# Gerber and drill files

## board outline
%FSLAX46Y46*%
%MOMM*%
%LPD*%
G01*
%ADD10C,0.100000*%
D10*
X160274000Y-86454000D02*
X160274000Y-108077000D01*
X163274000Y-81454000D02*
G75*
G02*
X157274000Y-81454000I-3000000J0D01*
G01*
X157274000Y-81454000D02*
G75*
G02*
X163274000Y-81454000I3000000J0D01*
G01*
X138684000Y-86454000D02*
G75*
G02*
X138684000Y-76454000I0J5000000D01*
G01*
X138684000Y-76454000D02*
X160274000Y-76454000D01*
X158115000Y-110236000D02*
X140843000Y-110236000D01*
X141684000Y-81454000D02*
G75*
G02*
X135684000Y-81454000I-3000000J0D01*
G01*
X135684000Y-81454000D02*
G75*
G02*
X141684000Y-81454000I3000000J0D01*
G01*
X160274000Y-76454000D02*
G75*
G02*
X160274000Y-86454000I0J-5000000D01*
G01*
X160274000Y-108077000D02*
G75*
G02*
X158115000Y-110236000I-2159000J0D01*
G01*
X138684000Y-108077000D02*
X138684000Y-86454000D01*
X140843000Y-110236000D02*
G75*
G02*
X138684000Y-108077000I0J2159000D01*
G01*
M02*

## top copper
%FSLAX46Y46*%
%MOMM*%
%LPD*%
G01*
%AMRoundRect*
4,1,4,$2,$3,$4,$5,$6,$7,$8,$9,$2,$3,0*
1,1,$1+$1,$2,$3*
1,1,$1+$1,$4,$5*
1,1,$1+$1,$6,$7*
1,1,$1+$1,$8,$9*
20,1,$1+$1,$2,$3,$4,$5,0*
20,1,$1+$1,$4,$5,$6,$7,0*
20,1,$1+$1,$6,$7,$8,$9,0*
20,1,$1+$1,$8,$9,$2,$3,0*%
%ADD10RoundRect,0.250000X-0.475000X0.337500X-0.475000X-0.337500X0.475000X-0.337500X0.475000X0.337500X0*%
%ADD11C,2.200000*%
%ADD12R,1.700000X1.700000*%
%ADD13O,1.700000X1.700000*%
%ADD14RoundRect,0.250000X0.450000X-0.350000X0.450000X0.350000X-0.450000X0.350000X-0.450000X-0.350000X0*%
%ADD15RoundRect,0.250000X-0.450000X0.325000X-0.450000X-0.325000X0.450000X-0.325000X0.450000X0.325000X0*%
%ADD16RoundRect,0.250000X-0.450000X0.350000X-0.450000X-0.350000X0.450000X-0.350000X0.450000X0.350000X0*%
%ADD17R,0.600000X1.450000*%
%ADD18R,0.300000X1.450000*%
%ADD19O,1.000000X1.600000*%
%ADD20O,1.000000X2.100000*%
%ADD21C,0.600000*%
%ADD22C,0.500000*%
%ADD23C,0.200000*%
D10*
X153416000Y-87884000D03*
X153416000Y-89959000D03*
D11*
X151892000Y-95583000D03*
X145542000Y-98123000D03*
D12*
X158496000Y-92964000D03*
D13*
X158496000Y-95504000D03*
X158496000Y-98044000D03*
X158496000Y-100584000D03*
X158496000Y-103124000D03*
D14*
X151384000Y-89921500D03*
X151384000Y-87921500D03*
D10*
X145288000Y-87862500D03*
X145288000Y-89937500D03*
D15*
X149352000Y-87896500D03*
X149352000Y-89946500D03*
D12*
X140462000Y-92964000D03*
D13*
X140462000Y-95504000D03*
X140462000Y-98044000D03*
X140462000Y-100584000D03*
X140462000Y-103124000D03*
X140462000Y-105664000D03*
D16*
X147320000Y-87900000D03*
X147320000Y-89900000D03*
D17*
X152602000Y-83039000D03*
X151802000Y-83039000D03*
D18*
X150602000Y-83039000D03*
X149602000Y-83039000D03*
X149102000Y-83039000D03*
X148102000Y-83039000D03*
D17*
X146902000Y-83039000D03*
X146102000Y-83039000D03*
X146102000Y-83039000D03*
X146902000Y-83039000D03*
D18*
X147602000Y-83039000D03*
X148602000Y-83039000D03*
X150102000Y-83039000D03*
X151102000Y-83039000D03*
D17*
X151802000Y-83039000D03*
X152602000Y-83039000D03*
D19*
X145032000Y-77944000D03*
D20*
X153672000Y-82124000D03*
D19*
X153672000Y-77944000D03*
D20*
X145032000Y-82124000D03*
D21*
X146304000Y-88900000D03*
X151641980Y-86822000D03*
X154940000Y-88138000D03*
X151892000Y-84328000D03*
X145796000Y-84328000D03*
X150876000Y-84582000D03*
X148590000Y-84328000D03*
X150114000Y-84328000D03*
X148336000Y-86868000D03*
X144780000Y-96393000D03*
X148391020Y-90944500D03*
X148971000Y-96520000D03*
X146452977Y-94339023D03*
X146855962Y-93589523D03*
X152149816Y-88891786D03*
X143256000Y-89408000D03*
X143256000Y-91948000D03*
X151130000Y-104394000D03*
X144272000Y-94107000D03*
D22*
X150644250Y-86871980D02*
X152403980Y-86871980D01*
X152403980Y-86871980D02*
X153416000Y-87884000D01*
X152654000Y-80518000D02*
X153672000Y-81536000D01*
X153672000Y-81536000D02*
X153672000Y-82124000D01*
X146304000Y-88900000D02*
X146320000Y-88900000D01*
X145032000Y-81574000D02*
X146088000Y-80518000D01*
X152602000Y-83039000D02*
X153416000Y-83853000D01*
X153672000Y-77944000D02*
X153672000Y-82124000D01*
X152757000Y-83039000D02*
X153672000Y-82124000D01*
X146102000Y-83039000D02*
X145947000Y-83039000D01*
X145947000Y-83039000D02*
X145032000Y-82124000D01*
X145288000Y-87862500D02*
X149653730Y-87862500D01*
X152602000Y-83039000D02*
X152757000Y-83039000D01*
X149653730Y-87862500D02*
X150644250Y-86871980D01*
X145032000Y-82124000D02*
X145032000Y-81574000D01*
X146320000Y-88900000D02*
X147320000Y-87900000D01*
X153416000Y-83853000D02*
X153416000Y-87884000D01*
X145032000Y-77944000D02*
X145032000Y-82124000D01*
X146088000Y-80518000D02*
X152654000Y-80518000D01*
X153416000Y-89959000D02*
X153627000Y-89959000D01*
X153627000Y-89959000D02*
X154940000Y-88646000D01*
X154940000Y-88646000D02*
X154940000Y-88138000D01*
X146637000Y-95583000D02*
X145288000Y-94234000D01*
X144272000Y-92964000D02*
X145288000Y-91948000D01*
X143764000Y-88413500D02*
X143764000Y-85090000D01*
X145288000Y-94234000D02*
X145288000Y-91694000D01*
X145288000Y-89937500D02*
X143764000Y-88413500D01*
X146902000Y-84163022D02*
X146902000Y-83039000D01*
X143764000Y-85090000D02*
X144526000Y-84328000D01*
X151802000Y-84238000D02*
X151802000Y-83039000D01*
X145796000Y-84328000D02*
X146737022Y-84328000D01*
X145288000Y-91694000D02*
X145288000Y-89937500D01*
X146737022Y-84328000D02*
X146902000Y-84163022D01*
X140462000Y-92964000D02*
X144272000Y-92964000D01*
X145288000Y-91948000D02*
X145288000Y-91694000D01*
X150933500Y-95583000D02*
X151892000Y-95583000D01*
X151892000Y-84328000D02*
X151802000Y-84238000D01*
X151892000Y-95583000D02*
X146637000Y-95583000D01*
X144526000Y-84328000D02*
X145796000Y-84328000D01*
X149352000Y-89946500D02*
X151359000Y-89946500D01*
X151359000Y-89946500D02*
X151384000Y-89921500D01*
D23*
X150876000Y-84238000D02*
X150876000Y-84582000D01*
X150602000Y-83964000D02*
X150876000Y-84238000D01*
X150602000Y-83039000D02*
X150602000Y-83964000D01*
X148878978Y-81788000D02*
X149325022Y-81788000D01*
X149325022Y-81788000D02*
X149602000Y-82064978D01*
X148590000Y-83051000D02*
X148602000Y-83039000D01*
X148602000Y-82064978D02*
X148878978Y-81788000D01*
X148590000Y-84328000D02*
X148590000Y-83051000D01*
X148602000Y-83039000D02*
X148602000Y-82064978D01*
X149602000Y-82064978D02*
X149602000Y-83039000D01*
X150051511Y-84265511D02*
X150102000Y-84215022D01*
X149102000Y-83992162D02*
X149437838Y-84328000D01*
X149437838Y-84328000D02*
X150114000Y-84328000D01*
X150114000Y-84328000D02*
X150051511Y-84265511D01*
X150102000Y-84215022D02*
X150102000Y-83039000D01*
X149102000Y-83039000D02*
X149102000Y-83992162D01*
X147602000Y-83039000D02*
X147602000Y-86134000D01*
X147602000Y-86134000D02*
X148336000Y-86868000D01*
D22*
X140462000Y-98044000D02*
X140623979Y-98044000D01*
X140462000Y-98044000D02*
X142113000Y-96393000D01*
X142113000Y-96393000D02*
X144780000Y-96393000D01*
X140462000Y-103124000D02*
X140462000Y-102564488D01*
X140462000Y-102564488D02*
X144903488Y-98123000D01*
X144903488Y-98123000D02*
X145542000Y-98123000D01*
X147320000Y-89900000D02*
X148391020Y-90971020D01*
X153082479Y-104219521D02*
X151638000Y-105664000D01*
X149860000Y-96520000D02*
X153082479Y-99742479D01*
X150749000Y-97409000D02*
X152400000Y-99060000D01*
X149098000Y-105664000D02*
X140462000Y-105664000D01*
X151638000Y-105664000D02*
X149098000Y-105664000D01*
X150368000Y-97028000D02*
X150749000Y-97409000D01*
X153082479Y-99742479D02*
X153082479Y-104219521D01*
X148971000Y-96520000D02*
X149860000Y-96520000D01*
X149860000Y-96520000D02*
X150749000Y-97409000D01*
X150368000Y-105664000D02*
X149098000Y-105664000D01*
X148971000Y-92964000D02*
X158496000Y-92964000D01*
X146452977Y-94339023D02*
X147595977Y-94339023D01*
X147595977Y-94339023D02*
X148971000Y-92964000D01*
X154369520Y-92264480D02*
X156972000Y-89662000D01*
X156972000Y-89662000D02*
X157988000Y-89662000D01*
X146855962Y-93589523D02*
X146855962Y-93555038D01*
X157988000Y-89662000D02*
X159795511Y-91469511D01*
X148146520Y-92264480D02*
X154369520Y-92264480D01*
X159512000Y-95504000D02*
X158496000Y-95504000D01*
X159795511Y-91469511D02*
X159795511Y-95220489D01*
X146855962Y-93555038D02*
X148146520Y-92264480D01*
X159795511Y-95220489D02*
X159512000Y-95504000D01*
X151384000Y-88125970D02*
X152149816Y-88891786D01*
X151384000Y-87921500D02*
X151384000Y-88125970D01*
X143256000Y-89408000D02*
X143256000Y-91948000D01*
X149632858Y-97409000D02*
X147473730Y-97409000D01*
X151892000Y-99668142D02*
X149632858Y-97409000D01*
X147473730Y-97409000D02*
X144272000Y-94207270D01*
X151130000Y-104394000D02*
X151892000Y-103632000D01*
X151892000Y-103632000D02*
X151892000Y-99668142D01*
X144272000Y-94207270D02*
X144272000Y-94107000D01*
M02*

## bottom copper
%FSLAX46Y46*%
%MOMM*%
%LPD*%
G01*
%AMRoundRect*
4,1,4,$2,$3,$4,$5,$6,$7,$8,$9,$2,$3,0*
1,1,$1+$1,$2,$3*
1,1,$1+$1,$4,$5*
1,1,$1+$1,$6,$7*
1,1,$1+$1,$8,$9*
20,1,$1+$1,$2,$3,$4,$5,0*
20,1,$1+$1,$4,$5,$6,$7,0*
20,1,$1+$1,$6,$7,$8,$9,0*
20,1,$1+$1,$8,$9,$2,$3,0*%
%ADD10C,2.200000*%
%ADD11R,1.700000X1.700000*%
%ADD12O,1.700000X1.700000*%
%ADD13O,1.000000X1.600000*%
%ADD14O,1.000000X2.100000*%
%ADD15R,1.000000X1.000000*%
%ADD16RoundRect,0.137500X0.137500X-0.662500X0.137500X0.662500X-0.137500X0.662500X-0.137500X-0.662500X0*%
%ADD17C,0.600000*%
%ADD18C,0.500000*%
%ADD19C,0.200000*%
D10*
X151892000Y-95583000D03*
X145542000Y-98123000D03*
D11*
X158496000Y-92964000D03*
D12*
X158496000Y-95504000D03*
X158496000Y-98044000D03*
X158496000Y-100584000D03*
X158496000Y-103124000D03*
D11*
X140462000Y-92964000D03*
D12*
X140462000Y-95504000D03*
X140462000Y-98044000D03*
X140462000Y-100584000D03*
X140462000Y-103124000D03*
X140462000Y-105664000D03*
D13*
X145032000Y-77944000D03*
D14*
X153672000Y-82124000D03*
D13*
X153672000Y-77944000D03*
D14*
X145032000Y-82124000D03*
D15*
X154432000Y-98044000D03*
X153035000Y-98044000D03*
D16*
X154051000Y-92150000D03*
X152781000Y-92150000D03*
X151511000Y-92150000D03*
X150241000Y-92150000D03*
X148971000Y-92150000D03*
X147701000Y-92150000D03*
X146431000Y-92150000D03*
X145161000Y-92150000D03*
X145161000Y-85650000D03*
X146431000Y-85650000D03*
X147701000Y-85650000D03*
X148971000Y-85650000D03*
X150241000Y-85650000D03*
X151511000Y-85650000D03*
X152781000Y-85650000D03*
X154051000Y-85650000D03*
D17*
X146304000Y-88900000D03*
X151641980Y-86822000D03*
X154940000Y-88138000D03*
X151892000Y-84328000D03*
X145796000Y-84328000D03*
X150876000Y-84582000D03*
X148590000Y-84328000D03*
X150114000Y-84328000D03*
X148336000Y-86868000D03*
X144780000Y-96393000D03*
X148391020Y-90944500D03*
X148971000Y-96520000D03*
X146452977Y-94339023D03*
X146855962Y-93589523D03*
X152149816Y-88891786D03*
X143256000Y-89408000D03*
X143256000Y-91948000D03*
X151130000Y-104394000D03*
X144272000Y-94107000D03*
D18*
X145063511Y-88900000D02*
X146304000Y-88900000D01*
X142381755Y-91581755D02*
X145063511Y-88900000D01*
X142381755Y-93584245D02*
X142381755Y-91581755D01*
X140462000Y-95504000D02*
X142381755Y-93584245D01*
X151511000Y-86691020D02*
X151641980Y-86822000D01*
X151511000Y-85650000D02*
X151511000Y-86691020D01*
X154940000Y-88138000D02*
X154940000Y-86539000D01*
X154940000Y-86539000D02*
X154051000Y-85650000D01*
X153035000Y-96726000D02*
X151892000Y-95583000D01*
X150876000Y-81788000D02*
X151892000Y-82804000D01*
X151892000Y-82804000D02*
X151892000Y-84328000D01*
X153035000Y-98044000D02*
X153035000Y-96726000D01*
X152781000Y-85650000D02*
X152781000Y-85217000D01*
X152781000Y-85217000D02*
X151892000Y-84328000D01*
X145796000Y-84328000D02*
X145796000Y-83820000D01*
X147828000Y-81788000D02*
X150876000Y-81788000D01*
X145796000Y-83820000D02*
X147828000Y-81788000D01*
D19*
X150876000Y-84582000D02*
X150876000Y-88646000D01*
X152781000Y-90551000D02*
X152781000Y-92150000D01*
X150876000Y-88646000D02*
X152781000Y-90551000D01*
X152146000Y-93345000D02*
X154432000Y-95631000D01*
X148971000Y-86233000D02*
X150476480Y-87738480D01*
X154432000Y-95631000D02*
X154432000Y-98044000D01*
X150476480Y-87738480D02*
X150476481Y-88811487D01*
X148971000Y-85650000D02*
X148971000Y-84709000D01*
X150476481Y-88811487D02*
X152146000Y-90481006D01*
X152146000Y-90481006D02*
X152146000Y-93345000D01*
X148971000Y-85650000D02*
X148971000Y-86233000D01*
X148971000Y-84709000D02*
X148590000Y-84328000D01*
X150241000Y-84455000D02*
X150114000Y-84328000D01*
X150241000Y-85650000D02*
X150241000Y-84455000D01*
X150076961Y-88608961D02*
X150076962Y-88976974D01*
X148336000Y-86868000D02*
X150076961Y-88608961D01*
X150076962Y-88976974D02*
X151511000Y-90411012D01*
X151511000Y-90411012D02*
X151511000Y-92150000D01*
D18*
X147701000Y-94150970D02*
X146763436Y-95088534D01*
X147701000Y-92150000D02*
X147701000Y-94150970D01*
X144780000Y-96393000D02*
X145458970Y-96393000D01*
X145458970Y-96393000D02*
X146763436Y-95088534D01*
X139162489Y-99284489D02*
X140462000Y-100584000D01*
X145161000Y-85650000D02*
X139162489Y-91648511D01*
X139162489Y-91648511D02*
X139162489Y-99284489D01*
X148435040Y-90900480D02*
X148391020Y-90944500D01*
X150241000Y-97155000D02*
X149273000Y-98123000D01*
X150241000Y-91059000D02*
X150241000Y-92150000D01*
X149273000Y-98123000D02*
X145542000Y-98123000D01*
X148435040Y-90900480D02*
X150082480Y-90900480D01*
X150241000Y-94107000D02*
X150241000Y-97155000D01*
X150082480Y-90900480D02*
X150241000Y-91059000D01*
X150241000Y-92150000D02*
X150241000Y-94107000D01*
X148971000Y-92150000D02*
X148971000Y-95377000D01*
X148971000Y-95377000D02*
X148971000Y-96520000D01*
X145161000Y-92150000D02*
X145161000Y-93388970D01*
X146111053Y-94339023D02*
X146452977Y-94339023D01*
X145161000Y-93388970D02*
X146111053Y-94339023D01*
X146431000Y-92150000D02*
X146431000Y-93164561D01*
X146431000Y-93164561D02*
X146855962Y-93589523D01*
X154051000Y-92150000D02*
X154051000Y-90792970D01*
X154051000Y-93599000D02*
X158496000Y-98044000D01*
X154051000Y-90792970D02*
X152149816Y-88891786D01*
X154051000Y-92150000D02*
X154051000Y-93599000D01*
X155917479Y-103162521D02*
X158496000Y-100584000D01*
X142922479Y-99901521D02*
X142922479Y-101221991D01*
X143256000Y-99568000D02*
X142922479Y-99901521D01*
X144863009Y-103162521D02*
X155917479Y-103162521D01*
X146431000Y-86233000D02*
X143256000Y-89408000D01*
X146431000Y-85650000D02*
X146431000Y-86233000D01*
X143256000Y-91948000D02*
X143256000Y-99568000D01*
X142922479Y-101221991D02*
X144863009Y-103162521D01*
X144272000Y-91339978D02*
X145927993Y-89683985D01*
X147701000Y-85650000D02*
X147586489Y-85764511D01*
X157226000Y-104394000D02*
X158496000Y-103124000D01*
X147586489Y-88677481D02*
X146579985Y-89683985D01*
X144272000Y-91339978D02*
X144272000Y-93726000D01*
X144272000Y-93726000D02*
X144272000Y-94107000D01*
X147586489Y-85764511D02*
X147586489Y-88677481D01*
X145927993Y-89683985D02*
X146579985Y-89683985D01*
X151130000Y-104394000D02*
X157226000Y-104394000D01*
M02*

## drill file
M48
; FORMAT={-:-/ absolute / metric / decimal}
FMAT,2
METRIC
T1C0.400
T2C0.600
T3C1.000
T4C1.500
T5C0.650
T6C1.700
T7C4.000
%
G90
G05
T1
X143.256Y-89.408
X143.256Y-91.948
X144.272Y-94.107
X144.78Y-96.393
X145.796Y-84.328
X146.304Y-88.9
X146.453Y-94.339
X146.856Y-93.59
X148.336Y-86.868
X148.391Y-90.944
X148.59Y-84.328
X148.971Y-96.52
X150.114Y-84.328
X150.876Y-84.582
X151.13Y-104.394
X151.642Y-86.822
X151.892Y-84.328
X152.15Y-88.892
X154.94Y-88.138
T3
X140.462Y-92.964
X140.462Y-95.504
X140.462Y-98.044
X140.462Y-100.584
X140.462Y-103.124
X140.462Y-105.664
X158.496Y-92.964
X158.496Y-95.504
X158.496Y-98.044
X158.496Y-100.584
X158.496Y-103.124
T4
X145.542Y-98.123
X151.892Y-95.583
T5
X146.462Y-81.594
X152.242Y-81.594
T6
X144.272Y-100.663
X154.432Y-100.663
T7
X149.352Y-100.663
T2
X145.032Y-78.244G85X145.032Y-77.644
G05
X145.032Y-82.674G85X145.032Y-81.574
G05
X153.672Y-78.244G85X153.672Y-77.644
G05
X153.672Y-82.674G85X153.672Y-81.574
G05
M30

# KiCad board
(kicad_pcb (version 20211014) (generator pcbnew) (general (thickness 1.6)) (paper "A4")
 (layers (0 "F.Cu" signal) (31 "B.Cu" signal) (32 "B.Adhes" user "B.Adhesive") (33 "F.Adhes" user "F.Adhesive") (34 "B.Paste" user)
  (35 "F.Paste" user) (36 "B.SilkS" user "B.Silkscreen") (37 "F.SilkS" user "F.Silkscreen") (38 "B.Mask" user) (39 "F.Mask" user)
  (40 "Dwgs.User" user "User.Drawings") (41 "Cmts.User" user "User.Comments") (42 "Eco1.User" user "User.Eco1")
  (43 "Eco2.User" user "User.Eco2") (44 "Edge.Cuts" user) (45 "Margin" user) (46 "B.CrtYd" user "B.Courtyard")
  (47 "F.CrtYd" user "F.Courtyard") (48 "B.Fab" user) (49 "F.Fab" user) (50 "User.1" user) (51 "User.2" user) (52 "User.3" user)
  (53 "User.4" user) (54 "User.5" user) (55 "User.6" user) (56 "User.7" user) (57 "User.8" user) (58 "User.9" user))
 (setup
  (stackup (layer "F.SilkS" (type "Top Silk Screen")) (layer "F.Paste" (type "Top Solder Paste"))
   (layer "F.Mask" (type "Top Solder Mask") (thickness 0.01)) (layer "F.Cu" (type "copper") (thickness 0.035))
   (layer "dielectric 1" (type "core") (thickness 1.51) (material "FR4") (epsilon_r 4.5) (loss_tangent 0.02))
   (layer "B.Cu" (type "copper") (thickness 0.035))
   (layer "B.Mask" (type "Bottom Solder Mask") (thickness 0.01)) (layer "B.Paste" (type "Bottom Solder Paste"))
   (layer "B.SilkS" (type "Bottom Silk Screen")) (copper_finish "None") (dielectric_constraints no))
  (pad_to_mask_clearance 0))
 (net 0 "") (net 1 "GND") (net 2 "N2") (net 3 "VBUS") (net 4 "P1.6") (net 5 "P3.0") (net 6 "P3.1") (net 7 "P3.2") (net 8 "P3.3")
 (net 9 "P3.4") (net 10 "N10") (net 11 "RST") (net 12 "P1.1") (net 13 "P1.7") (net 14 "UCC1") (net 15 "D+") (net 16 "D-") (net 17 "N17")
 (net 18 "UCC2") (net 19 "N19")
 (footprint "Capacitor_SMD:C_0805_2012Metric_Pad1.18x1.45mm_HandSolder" (layer "F.Cu") (at 153.416 88.9215 -90)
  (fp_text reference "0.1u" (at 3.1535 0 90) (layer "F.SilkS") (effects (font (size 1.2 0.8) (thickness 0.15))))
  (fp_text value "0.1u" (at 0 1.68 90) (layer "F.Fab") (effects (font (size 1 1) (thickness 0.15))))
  (pad "1" smd roundrect (at -1.0375 0 270) (size 1.175 1.45) (layers "F.Cu" "F.Paste" "F.Mask") (roundrect_rratio 0.2127659574)
   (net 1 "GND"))
  (pad "2" smd roundrect (at 1.0375 0 270) (size 1.175 1.45) (layers "F.Cu" "F.Paste" "F.Mask") (roundrect_rratio 0.2127659574) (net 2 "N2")))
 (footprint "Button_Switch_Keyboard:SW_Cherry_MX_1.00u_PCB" (layer "F.Cu") (at 151.892 95.583)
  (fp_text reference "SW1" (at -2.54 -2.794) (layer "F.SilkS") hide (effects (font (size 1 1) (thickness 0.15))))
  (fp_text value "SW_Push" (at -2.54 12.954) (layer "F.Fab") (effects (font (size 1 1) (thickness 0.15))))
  (pad "" np_thru_hole circle (at -2.54 5.08) (size 4 4) (drill 4) (layers *.Cu *.Mask))
  (pad "" np_thru_hole circle (at -7.62 5.08) (size 1.7 1.7) (drill 1.7) (layers *.Cu *.Mask))
  (pad "" np_thru_hole circle (at 2.54 5.08) (size 1.7 1.7) (drill 1.7) (layers *.Cu *.Mask))
  (pad "1" thru_hole circle (at 0 0) (size 2.2 2.2) (drill 1.5) (layers *.Cu *.Mask) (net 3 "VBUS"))
  (pad "2" thru_hole circle (at -6.35 2.54) (size 2.2 2.2) (drill 1.5) (layers *.Cu *.Mask) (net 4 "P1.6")))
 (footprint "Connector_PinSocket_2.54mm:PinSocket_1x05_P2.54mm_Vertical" (layer "F.Cu") (at 158.496 92.964)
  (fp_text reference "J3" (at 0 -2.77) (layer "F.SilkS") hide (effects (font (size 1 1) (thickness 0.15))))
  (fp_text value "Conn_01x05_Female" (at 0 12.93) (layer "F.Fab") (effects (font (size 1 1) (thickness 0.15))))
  (pad "1" thru_hole rect (at 0 0) (size 1.7 1.7) (drill 1) (layers *.Cu *.Mask) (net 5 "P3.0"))
  (pad "2" thru_hole oval (at 0 2.54) (size 1.7 1.7) (drill 1) (layers *.Cu *.Mask) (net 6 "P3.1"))
  (pad "3" thru_hole oval (at 0 5.08) (size 1.7 1.7) (drill 1) (layers *.Cu *.Mask) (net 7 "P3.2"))
  (pad "4" thru_hole oval (at 0 7.62) (size 1.7 1.7) (drill 1) (layers *.Cu *.Mask) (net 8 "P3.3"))
  (pad "5" thru_hole oval (at 0 10.16) (size 1.7 1.7) (drill 1) (layers *.Cu *.Mask) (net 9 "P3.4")))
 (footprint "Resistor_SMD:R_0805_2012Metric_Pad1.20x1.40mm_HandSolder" (layer "F.Cu") (at 151.384 88.9215 90)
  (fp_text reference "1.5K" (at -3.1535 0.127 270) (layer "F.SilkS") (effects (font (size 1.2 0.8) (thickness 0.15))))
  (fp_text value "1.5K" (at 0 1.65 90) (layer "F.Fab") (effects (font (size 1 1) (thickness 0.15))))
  (pad "1" smd roundrect (at -1 0 90) (size 1.2 1.4) (layers "F.Cu" "F.Paste" "F.Mask") (roundrect_rratio 0.2083333333) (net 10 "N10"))
  (pad "2" smd roundrect (at 1 0 90) (size 1.2 1.4) (layers "F.Cu" "F.Paste" "F.Mask") (roundrect_rratio 0.2083333333) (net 7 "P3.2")))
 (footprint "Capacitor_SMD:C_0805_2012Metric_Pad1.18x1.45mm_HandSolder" (layer "F.Cu") (at 145.288 88.9 -90)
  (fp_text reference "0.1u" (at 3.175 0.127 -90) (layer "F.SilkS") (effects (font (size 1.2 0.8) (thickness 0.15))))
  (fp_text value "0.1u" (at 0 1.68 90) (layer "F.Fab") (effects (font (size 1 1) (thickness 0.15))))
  (pad "1" smd roundrect (at -1.0375 0 270) (size 1.175 1.45) (layers "F.Cu" "F.Paste" "F.Mask") (roundrect_rratio 0.2127659574)
   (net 1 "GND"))
  (pad "2" smd roundrect (at 1.0375 0 270) (size 1.175 1.45) (layers "F.Cu" "F.Paste" "F.Mask") (roundrect_rratio 0.2127659574)
   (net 3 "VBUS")))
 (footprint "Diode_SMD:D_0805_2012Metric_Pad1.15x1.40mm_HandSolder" (layer "F.Cu") (at 149.352 88.9215 -90)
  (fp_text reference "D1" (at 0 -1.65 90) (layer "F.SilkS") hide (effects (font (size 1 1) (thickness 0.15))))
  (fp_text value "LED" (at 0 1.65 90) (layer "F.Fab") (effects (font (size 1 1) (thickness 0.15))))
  (pad "1" smd roundrect (at -1.025 0 270) (size 1.15 1.4) (layers "F.Cu" "F.Paste" "F.Mask") (roundrect_rratio 0.2173913043) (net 1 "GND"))
  (pad "2" smd roundrect (at 1.025 0 270) (size 1.15 1.4) (layers "F.Cu" "F.Paste" "F.Mask") (roundrect_rratio 0.2173913043) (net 10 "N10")))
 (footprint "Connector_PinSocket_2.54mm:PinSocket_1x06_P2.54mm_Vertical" (layer "F.Cu") (at 140.462 92.964)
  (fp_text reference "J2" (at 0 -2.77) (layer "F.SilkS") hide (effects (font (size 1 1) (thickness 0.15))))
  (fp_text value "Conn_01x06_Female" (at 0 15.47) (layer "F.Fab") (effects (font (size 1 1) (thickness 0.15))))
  (pad "1" thru_hole rect (at 0 0) (size 1.7 1.7) (drill 1) (layers *.Cu *.Mask) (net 3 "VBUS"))
  (pad "2" thru_hole oval (at 0 2.54) (size 1.7 1.7) (drill 1) (layers *.Cu *.Mask) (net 1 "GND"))
  (pad "3" thru_hole oval (at 0 5.08) (size 1.7 1.7) (drill 1) (layers *.Cu *.Mask) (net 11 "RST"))
  (pad "4" thru_hole oval (at 0 7.62) (size 1.7 1.7) (drill 1) (layers *.Cu *.Mask) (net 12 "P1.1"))
  (pad "5" thru_hole oval (at 0 10.16) (size 1.7 1.7) (drill 1) (layers *.Cu *.Mask) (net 4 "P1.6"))
  (pad "6" thru_hole oval (at 0 12.7) (size 1.7 1.7) (drill 1) (layers *.Cu *.Mask) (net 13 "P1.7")))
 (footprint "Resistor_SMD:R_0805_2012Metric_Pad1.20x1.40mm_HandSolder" (layer "F.Cu") (at 147.32 88.9 -90)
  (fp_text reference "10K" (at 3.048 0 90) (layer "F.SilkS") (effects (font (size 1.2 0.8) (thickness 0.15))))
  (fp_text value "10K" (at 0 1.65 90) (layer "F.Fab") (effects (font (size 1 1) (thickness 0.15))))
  (pad "1" smd roundrect (at -1 0 270) (size 1.2 1.4) (layers "F.Cu" "F.Paste" "F.Mask") (roundrect_rratio 0.2083333333) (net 1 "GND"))
  (pad "2" smd roundrect (at 1 0 270) (size 1.2 1.4) (layers "F.Cu" "F.Paste" "F.Mask") (roundrect_rratio 0.2083333333) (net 4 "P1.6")))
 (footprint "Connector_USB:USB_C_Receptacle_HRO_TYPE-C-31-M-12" (layer "F.Cu") (at 149.352 78.994 180)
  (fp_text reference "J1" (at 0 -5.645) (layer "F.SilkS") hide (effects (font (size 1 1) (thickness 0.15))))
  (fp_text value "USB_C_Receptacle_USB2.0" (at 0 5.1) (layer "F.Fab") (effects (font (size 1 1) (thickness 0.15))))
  (pad "" np_thru_hole circle (at 2.89 -2.6 180) (size 0.65 0.65) (drill 0.65) (layers *.Cu *.Mask))
  (pad "" np_thru_hole circle (at -2.89 -2.6 180) (size 0.65 0.65) (drill 0.65) (layers *.Cu *.Mask))
  (pad "A1" smd rect (at -3.25 -4.045 180) (size 0.6 1.45) (layers "F.Cu" "F.Paste" "F.Mask") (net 1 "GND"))
  (pad "A4" smd rect (at -2.45 -4.045 180) (size 0.6 1.45) (layers "F.Cu" "F.Paste" "F.Mask") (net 3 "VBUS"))
  (pad "A5" smd rect (at -1.25 -4.045 180) (size 0.3 1.45) (layers "F.Cu" "F.Paste" "F.Mask") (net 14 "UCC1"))
  (pad "A6" smd rect (at -0.25 -4.045 180) (size 0.3 1.45) (layers "F.Cu" "F.Paste" "F.Mask") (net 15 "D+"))
  (pad "A7" smd rect (at 0.25 -4.045 180) (size 0.3 1.45) (layers "F.Cu" "F.Paste" "F.Mask") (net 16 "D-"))
  (pad "A8" smd rect (at 1.25 -4.045 180) (size 0.3 1.45) (layers "F.Cu" "F.Paste" "F.Mask") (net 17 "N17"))
  (pad "A9" smd rect (at 2.45 -4.045 180) (size 0.6 1.45) (layers "F.Cu" "F.Paste" "F.Mask") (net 3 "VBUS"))
  (pad "A12" smd rect (at 3.25 -4.045 180) (size 0.6 1.45) (layers "F.Cu" "F.Paste" "F.Mask") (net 1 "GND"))
  (pad "B1" smd rect (at 3.25 -4.045 180) (size 0.6 1.45) (layers "F.Cu" "F.Paste" "F.Mask") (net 1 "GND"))
  (pad "B4" smd rect (at 2.45 -4.045 180) (size 0.6 1.45) (layers "F.Cu" "F.Paste" "F.Mask") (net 3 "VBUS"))
  (pad "B5" smd rect (at 1.75 -4.045 180) (size 0.3 1.45) (layers "F.Cu" "F.Paste" "F.Mask") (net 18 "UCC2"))
  (pad "B6" smd rect (at 0.75 -4.045 180) (size 0.3 1.45) (layers "F.Cu" "F.Paste" "F.Mask") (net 15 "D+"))
  (pad "B7" smd rect (at -0.75 -4.045 180) (size 0.3 1.45) (layers "F.Cu" "F.Paste" "F.Mask") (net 16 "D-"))
  (pad "B8" smd rect (at -1.75 -4.045 180) (size 0.3 1.45) (layers "F.Cu" "F.Paste" "F.Mask") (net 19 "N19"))
  (pad "B9" smd rect (at -2.45 -4.045 180) (size 0.6 1.45) (layers "F.Cu" "F.Paste" "F.Mask") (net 3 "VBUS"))
  (pad "B12" smd rect (at -3.25 -4.045 180) (size 0.6 1.45) (layers "F.Cu" "F.Paste" "F.Mask") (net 1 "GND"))
  (pad "S1" thru_hole oval (at 4.32 1.05 180) (size 1 1.6) (drill oval 0.6 1.2) (layers *.Cu *.Mask) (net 1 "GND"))
  (pad "S1" thru_hole oval (at -4.32 -3.13 180) (size 1 2.1) (drill oval 0.6 1.7) (layers *.Cu *.Mask) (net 1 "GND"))
  (pad "S1" thru_hole oval (at -4.32 1.05 180) (size 1 1.6) (drill oval 0.6 1.2) (layers *.Cu *.Mask) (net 1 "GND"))
  (pad "S1" thru_hole oval (at 4.32 -3.13 180) (size 1 2.1) (drill oval 0.6 1.7) (layers *.Cu *.Mask) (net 1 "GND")))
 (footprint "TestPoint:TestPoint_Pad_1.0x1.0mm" (layer "B.Cu") (at 154.432 98.044 180)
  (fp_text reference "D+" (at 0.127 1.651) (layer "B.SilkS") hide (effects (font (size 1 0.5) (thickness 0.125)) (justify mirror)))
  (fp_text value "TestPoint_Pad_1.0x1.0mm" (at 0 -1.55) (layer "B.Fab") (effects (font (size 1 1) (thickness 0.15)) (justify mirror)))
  (pad "1" smd rect (at 0 0 180) (size 1 1) (layers "B.Cu" "B.Mask") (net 15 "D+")))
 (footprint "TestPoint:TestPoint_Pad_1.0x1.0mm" (layer "B.Cu") (at 153.035 98.044 180)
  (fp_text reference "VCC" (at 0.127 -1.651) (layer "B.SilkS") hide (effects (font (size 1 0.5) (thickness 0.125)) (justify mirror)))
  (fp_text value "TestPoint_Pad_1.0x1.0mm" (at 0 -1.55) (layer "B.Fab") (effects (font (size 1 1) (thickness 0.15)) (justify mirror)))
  (pad "1" smd rect (at 0 0 180) (size 1 1) (layers "B.Cu" "B.Mask") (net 3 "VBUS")))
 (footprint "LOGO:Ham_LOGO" (layer "B.Cu") (at 143.859 103.378 180)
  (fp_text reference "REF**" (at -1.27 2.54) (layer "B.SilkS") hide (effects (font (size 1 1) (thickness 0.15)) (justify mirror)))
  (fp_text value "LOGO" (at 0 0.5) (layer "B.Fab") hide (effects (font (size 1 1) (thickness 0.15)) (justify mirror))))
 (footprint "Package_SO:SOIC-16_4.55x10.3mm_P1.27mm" (layer "B.Cu") (at 149.606 88.9 90)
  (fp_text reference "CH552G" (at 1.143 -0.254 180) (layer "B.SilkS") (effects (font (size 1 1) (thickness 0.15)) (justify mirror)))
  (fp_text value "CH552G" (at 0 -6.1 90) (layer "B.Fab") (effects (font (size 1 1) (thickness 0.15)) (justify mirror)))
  (pad "1" smd roundrect (at -3.25 4.445 90) (size 1.6 0.55) (layers "B.Cu" "B.Paste" "B.Mask") (roundrect_rratio 0.25) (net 7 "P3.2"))
  (pad "2" smd roundrect (at -3.25 3.175 90) (size 1.6 0.55) (layers "B.Cu" "B.Paste" "B.Mask") (roundrect_rratio 0.25) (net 14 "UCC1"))
  (pad "3" smd roundrect (at -3.25 1.905 90) (size 1.6 0.55) (layers "B.Cu" "B.Paste" "B.Mask") (roundrect_rratio 0.25) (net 18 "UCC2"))
  (pad "4" smd roundrect (at -3.25 0.635 90) (size 1.6 0.55) (layers "B.Cu" "B.Paste" "B.Mask") (roundrect_rratio 0.25) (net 4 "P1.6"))
  (pad "5" smd roundrect (at -3.25 -0.635 90) (size 1.6 0.55) (layers "B.Cu" "B.Paste" "B.Mask") (roundrect_rratio 0.25) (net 13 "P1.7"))
  (pad "6" smd roundrect (at -3.25 -1.905 90) (size 1.6 0.55) (layers "B.Cu" "B.Paste" "B.Mask") (roundrect_rratio 0.25) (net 11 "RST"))
  (pad "7" smd roundrect (at -3.25 -3.175 90) (size 1.6 0.55) (layers "B.Cu" "B.Paste" "B.Mask") (roundrect_rratio 0.25) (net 6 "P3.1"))
  (pad "8" smd roundrect (at -3.25 -4.445 90) (size 1.6 0.55) (layers "B.Cu" "B.Paste" "B.Mask") (roundrect_rratio 0.25) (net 5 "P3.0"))
  (pad "9" smd roundrect (at 3.25 -4.445 90) (size 1.6 0.55) (layers "B.Cu" "B.Paste" "B.Mask") (roundrect_rratio 0.25) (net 12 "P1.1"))
  (pad "10" smd roundrect (at 3.25 -3.175 90) (size 1.6 0.55) (layers "B.Cu" "B.Paste" "B.Mask") (roundrect_rratio 0.25) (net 8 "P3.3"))
  (pad "11" smd roundrect (at 3.25 -1.905 90) (size 1.6 0.55) (layers "B.Cu" "B.Paste" "B.Mask") (roundrect_rratio 0.25) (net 9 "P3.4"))
  (pad "12" smd roundrect (at 3.25 -0.635 90) (size 1.6 0.55) (layers "B.Cu" "B.Paste" "B.Mask") (roundrect_rratio 0.25) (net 15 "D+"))
  (pad "13" smd roundrect (at 3.25 0.635 90) (size 1.6 0.55) (layers "B.Cu" "B.Paste" "B.Mask") (roundrect_rratio 0.25) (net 16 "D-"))
  (pad "14" smd roundrect (at 3.25 1.905 90) (size 1.6 0.55) (layers "B.Cu" "B.Paste" "B.Mask") (roundrect_rratio 0.25) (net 1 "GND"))
  (pad "15" smd roundrect (at 3.25 3.175 90) (size 1.6 0.55) (layers "B.Cu" "B.Paste" "B.Mask") (roundrect_rratio 0.25) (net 3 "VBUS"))
  (pad "16" smd roundrect (at 3.25 4.445 90) (size 1.6 0.55) (layers "B.Cu" "B.Paste" "B.Mask") (roundrect_rratio 0.25) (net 2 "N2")))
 (gr_line (start 160.274 86.454) (end 160.274 108.077) (layer "Edge.Cuts") (width 0.1))
 (gr_circle (center 160.274 81.454) (end 163.274 81.454) (layer "Edge.Cuts") (width 0.1) (fill none))
 (gr_arc (start 138.684 86.454) (mid 133.684 81.454) (end 138.684 76.454) (layer "Edge.Cuts") (width 0.1))
 (gr_line (start 138.684 76.454) (end 160.274 76.454) (layer "Edge.Cuts") (width 0.1))
 (gr_line (start 158.115 110.236) (end 140.843 110.236) (layer "Edge.Cuts") (width 0.1))
 (gr_circle (center 138.684 81.454) (end 141.684 81.454) (layer "Edge.Cuts") (width 0.1) (fill none))
 (gr_arc (start 160.274 76.454) (mid 165.274 81.454) (end 160.274 86.454) (layer "Edge.Cuts") (width 0.1))
 (gr_arc (start 160.274 108.077) (mid 159.641644 109.603644) (end 158.115 110.236) (layer "Edge.Cuts") (width 0.1))
 (gr_line (start 138.684 108.077) (end 138.684 86.454) (layer "Edge.Cuts") (width 0.1))
 (gr_arc (start 140.843 110.236) (mid 139.316356 109.603644) (end 138.684 108.077) (layer "Edge.Cuts") (width 0.1))
 (segment (start 150.64425 86.87198) (end 152.40398 86.87198) (width 0.5) (layer "F.Cu") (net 1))
 (segment (start 152.40398 86.87198) (end 153.416 87.884) (width 0.5) (layer "F.Cu") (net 1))
 (segment (start 152.654 80.518) (end 153.672 81.536) (width 0.5) (layer "F.Cu") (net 1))
 (segment (start 153.672 81.536) (end 153.672 82.124) (width 0.5) (layer "F.Cu") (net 1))
 (segment (start 146.304 88.9) (end 146.32 88.9) (width 0.5) (layer "F.Cu") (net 1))
 (segment (start 145.032 81.574) (end 146.088 80.518) (width 0.5) (layer "F.Cu") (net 1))
 (segment (start 152.602 83.039) (end 153.416 83.853) (width 0.5) (layer "F.Cu") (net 1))
 (segment (start 153.672 77.944) (end 153.672 82.124) (width 0.5) (layer "F.Cu") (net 1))
 (segment (start 152.757 83.039) (end 153.672 82.124) (width 0.5) (layer "F.Cu") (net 1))
 (segment (start 146.102 83.039) (end 145.947 83.039) (width 0.5) (layer "F.Cu") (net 1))
 (segment (start 145.947 83.039) (end 145.032 82.124) (width 0.5) (layer "F.Cu") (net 1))
 (segment (start 145.288 87.8625) (end 149.65373 87.8625) (width 0.5) (layer "F.Cu") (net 1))
 (segment (start 152.602 83.039) (end 152.757 83.039) (width 0.5) (layer "F.Cu") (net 1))
 (segment (start 149.65373 87.8625) (end 150.64425 86.87198) (width 0.5) (layer "F.Cu") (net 1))
 (segment (start 145.032 82.124) (end 145.032 81.574) (width 0.5) (layer "F.Cu") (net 1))
 (segment (start 146.32 88.9) (end 147.32 87.9) (width 0.5) (layer "F.Cu") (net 1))
 (segment (start 153.416 83.853) (end 153.416 87.884) (width 0.5) (layer "F.Cu") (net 1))
 (segment (start 145.032 77.944) (end 145.032 82.124) (width 0.5) (layer "F.Cu") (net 1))
 (segment (start 146.088 80.518) (end 152.654 80.518) (width 0.5) (layer "F.Cu") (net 1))
 (via (at 146.304 88.9) (size 0.6) (drill 0.4) (layers "F.Cu" "B.Cu") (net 1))
 (via (at 151.64198 86.822) (size 0.6) (drill 0.4) (layers "F.Cu" "B.Cu") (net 1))
 (segment (start 145.063511 88.9) (end 146.304 88.9) (width 0.5) (layer "B.Cu") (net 1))
 (segment (start 142.381755 91.581755) (end 145.063511 88.9) (width 0.5) (layer "B.Cu") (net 1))
 (segment (start 142.381755 93.584245) (end 142.381755 91.581755) (width 0.5) (layer "B.Cu") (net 1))
 (segment (start 140.462 95.504) (end 142.381755 93.584245) (width 0.5) (layer "B.Cu") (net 1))
 (segment (start 151.511 86.69102) (end 151.64198 86.822) (width 0.5) (layer "B.Cu") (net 1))
 (segment (start 151.511 85.65) (end 151.511 86.69102) (width 0.5) (layer "B.Cu") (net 1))
 (segment (start 153.416 89.959) (end 153.627 89.959) (width 0.5) (layer "F.Cu") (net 2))
 (segment (start 153.627 89.959) (end 154.94 88.646) (width 0.5) (layer "F.Cu") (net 2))
 (segment (start 154.94 88.646) (end 154.94 88.138) (width 0.5) (layer "F.Cu") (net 2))
 (via (at 154.94 88.138) (size 0.6) (drill 0.4) (layers "F.Cu" "B.Cu") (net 2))
 (segment (start 154.94 88.138) (end 154.94 86.539) (width 0.5) (layer "B.Cu") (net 2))
 (segment (start 154.94 86.539) (end 154.051 85.65) (width 0.5) (layer "B.Cu") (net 2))
 (segment (start 146.637 95.583) (end 145.288 94.234) (width 0.5) (layer "F.Cu") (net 3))
 (segment (start 144.272 92.964) (end 145.288 91.948) (width 0.5) (layer "F.Cu") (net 3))
 (segment (start 143.764 88.4135) (end 143.764 85.09) (width 0.5) (layer "F.Cu") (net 3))
 (segment (start 145.288 94.234) (end 145.288 91.694) (width 0.5) (layer "F.Cu") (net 3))
 (segment (start 145.288 89.9375) (end 143.764 88.4135) (width 0.5) (layer "F.Cu") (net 3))
 (segment (start 146.902 84.163022) (end 146.902 83.039) (width 0.5) (layer "F.Cu") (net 3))
 (segment (start 143.764 85.09) (end 144.526 84.328) (width 0.5) (layer "F.Cu") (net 3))
 (segment (start 151.802 84.238) (end 151.802 83.039) (width 0.5) (layer "F.Cu") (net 3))
 (segment (start 145.796 84.328) (end 146.737022 84.328) (width 0.5) (layer "F.Cu") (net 3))
 (segment (start 145.288 91.694) (end 145.288 89.9375) (width 0.5) (layer "F.Cu") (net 3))
 (segment (start 146.737022 84.328) (end 146.902 84.163022) (width 0.5) (layer "F.Cu") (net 3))
 (segment (start 140.462 92.964) (end 144.272 92.964) (width 0.5) (layer "F.Cu") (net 3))
 (segment (start 145.288 91.948) (end 145.288 91.694) (width 0.5) (layer "F.Cu") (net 3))
 (segment (start 150.9335 95.583) (end 151.892 95.583) (width 0.5) (layer "F.Cu") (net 3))
 (segment (start 151.892 84.328) (end 151.802 84.238) (width 0.5) (layer "F.Cu") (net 3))
 (segment (start 151.892 95.583) (end 146.637 95.583) (width 0.5) (layer "F.Cu") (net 3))
 (segment (start 144.526 84.328) (end 145.796 84.328) (width 0.5) (layer "F.Cu") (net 3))
 (via (at 151.892 84.328) (size 0.6) (drill 0.4) (layers "F.Cu" "B.Cu") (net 3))
 (via (at 145.796 84.328) (size 0.6) (drill 0.4) (layers "F.Cu" "B.Cu") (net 3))
 (segment (start 153.035 96.726) (end 151.892 95.583) (width 0.5) (layer "B.Cu") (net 3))
 (segment (start 150.876 81.788) (end 151.892 82.804) (width 0.5) (layer "B.Cu") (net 3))
 (segment (start 151.892 82.804) (end 151.892 84.328) (width 0.5) (layer "B.Cu") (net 3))
 (segment (start 153.035 98.044) (end 153.035 96.726) (width 0.5) (layer "B.Cu") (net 3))
 (segment (start 152.781 85.65) (end 152.781 85.217) (width 0.5) (layer "B.Cu") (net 3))
 (segment (start 152.781 85.217) (end 151.892 84.328) (width 0.5) (layer "B.Cu") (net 3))
 (segment (start 145.796 84.328) (end 145.796 83.82) (width 0.5) (layer "B.Cu") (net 3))
 (segment (start 147.828 81.788) (end 150.876 81.788) (width 0.5) (layer "B.Cu") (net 3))
 (segment (start 145.796 83.82) (end 147.828 81.788) (width 0.5) (layer "B.Cu") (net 3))
 (segment (start 149.352 89.9465) (end 151.359 89.9465) (width 0.5) (layer "F.Cu") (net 10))
 (segment (start 151.359 89.9465) (end 151.384 89.9215) (width 0.5) (layer "F.Cu") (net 10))
 (segment (start 150.876 84.238) (end 150.876 84.582) (width 0.2) (layer "F.Cu") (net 14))
 (segment (start 150.602 83.964) (end 150.876 84.238) (width 0.2) (layer "F.Cu") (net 14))
 (segment (start 150.602 83.039) (end 150.602 83.964) (width 0.2) (layer "F.Cu") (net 14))
 (via (at 150.876 84.582) (size 0.6) (drill 0.4) (layers "F.Cu" "B.Cu") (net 14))
 (segment (start 150.876 84.582) (end 150.876 88.646) (width 0.2) (layer "B.Cu") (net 14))
 (segment (start 152.781 90.551) (end 152.781 92.15) (width 0.2) (layer "B.Cu") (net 14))
 (segment (start 150.876 88.646) (end 152.781 90.551) (width 0.2) (layer "B.Cu") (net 14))
 (segment (start 148.878978 81.788) (end 149.325022 81.788) (width 0.2) (layer "F.Cu") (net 15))
 (segment (start 149.325022 81.788) (end 149.602 82.064978) (width 0.2) (layer "F.Cu") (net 15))
 (segment (start 148.59 83.051) (end 148.602 83.039) (width 0.2) (layer "F.Cu") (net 15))
 (segment (start 148.602 82.064978) (end 148.878978 81.788) (width 0.2) (layer "F.Cu") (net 15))
 (segment (start 148.59 84.328) (end 148.59 83.051) (width 0.2) (layer "F.Cu") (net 15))
 (segment (start 148.602 83.039) (end 148.602 82.064978) (width 0.2) (layer "F.Cu") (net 15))
 (segment (start 149.602 82.064978) (end 149.602 83.039) (width 0.2) (layer "F.Cu") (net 15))
 (via (at 148.59 84.328) (size 0.6) (drill 0.4) (layers "F.Cu" "B.Cu") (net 15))
 (segment (start 152.146 93.345) (end 154.432 95.631) (width 0.2) (layer "B.Cu") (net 15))
 (segment (start 148.971 86.233) (end 150.47648 87.73848) (width 0.2) (layer "B.Cu") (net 15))
 (segment (start 154.432 95.631) (end 154.432 98.044) (width 0.2) (layer "B.Cu") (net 15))
 (segment (start 150.47648 87.73848) (end 150.476481 88.811487) (width 0.2) (layer "B.Cu") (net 15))
 (segment (start 148.971 85.65) (end 148.971 84.709) (width 0.2) (layer "B.Cu") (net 15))
 (segment (start 150.476481 88.811487) (end 152.146 90.481006) (width 0.2) (layer "B.Cu") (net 15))
 (segment (start 152.146 90.481006) (end 152.146 93.345) (width 0.2) (layer "B.Cu") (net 15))
 (segment (start 148.971 85.65) (end 148.971 86.233) (width 0.2) (layer "B.Cu") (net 15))
 (segment (start 148.971 84.709) (end 148.59 84.328) (width 0.2) (layer "B.Cu") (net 15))
 (segment (start 150.051511 84.265511) (end 150.102 84.215022) (width 0.2) (layer "F.Cu") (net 16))
 (segment (start 149.102 83.992162) (end 149.437838 84.328) (width 0.2) (layer "F.Cu") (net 16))
 (segment (start 149.437838 84.328) (end 150.114 84.328) (width 0.2) (layer "F.Cu") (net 16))
 (segment (start 150.114 84.328) (end 150.051511 84.265511) (width 0.2) (layer "F.Cu") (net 16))
 (segment (start 150.102 84.215022) (end 150.102 83.039) (width 0.2) (layer "F.Cu") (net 16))
 (segment (start 149.102 83.039) (end 149.102 83.992162) (width 0.2) (layer "F.Cu") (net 16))
 (via (at 150.114 84.328) (size 0.6) (drill 0.4) (layers "F.Cu" "B.Cu") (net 16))
 (segment (start 150.241 84.455) (end 150.114 84.328) (width 0.2) (layer "B.Cu") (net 16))
 (segment (start 150.241 85.65) (end 150.241 84.455) (width 0.2) (layer "B.Cu") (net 16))
 (segment (start 147.602 83.039) (end 147.602 86.134) (width 0.2) (layer "F.Cu") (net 18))
 (segment (start 147.602 86.134) (end 148.336 86.868) (width 0.2) (layer "F.Cu") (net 18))
 (via (at 148.336 86.868) (size 0.6) (drill 0.4) (layers "F.Cu" "B.Cu") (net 18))
 (segment (start 150.076961 88.608961) (end 150.076962 88.976974) (width 0.2) (layer "B.Cu") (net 18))
 (segment (start 148.336 86.868) (end 150.076961 88.608961) (width 0.2) (layer "B.Cu") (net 18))
 (segment (start 150.076962 88.976974) (end 151.511 90.411012) (width 0.2) (layer "B.Cu") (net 18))
 (segment (start 151.511 90.411012) (end 151.511 92.15) (width 0.2) (layer "B.Cu") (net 18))
 (segment (start 140.462 98.044) (end 140.623979 98.044) (width 0.5) (layer "F.Cu") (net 11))
 (segment (start 140.462 98.044) (end 142.113 96.393) (width 0.5) (layer "F.Cu") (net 11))
 (segment (start 142.113 96.393) (end 144.78 96.393) (width 0.5) (layer "F.Cu") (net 11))
 (via (at 144.78 96.393) (size 0.6) (drill 0.4) (layers "F.Cu" "B.Cu") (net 11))
 (segment (start 147.701 94.15097) (end 146.763436 95.088534) (width 0.5) (layer "B.Cu") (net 11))
 (segment (start 147.701 92.15) (end 147.701 94.15097) (width 0.5) (layer "B.Cu") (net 11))
 (segment (start 144.78 96.393) (end 145.45897 96.393) (width 0.5) (layer "B.Cu") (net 11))
 (segment (start 145.45897 96.393) (end 146.763436 95.088534) (width 0.5) (layer "B.Cu") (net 11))
 (segment (start 139.162489 99.284489) (end 140.462 100.584) (width 0.5) (layer "B.Cu") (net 12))
 (segment (start 145.161 85.65) (end 139.162489 91.648511) (width 0.5) (layer "B.Cu") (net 12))
 (segment (start 139.162489 91.648511) (end 139.162489 99.284489) (width 0.5) (layer "B.Cu") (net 12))
 (segment (start 140.462 103.124) (end 140.462 102.564488) (width 0.5) (layer "F.Cu") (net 4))
 (segment (start 140.462 102.564488) (end 144.903488 98.123) (width 0.5) (layer "F.Cu") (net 4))
 (segment (start 144.903488 98.123) (end 145.542 98.123) (width 0.5) (layer "F.Cu") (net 4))
 (segment (start 147.32 89.9) (end 148.39102 90.97102) (width 0.5) (layer "F.Cu") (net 4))
 (via (at 148.39102 90.9445) (size 0.6) (drill 0.4) (layers "F.Cu" "B.Cu") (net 4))
 (segment (start 148.43504 90.90048) (end 148.39102 90.9445) (width 0.5) (layer "B.Cu") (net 4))
 (segment (start 150.241 97.155) (end 149.273 98.123) (width 0.5) (layer "B.Cu") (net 4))
 (segment (start 150.241 91.059) (end 150.241 92.15) (width 0.5) (layer "B.Cu") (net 4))
 (segment (start 149.273 98.123) (end 145.542 98.123) (width 0.5) (layer "B.Cu") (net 4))
 (segment (start 148.43504 90.90048) (end 150.08248 90.90048) (width 0.5) (layer "B.Cu") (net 4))
 (segment (start 150.241 94.107) (end 150.241 97.155) (width 0.5) (layer "B.Cu") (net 4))
 (segment (start 150.08248 90.90048) (end 150.241 91.059) (width 0.5) (layer "B.Cu") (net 4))
 (segment (start 150.241 92.15) (end 150.241 94.107) (width 0.5) (layer "B.Cu") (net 4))
 (segment (start 153.082479 104.219521) (end 151.638 105.664) (width 0.5) (layer "F.Cu") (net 13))
 (segment (start 149.86 96.52) (end 153.082479 99.742479) (width 0.5) (layer "F.Cu") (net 13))
 (segment (start 150.749 97.409) (end 152.4 99.06) (width 0.5) (layer "F.Cu") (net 13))
 (segment (start 149.098 105.664) (end 140.462 105.664) (width 0.5) (layer "F.Cu") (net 13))
 (segment (start 151.638 105.664) (end 149.098 105.664) (width 0.5) (layer "F.Cu") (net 13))
 (segment (start 150.368 97.028) (end 150.749 97.409) (width 0.5) (layer "F.Cu") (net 13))
 (segment (start 153.082479 99.742479) (end 153.082479 104.219521) (width 0.5) (layer "F.Cu") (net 13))
 (segment (start 148.971 96.52) (end 149.86 96.52) (width 0.5) (layer "F.Cu") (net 13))
 (segment (start 149.86 96.52) (end 150.749 97.409) (width 0.5) (layer "F.Cu") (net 13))
 (segment (start 150.368 105.664) (end 149.098 105.664) (width 0.5) (layer "F.Cu") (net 13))
 (via (at 148.971 96.52) (size 0.6) (drill 0.4) (layers "F.Cu" "B.Cu") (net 13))
 (segment (start 148.971 92.15) (end 148.971 95.377) (width 0.5) (layer "B.Cu") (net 13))
 (segment (start 148.971 95.377) (end 148.971 96.52) (width 0.5) (layer "B.Cu") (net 13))
 (segment (start 148.971 92.964) (end 158.496 92.964) (width 0.5) (layer "F.Cu") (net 5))
 (segment (start 146.452977 94.339023) (end 147.595977 94.339023) (width 0.5) (layer "F.Cu") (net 5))
 (segment (start 147.595977 94.339023) (end 148.971 92.964) (width 0.5) (layer "F.Cu") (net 5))
 (via (at 146.452977 94.339023) (size 0.6) (drill 0.4) (layers "F.Cu" "B.Cu") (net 5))
 (segment (start 145.161 92.15) (end 145.161 93.38897) (width 0.5) (layer "B.Cu") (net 5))
 (segment (start 146.111053 94.339023) (end 146.452977 94.339023) (width 0.5) (layer "B.Cu") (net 5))
 (segment (start 145.161 93.38897) (end 146.111053 94.339023) (width 0.5) (layer "B.Cu") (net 5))
 (segment (start 154.36952 92.26448) (end 156.972 89.662) (width 0.5) (layer "F.Cu") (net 6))
 (segment (start 156.972 89.662) (end 157.988 89.662) (width 0.5) (layer "F.Cu") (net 6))
 (segment (start 146.855962 93.589523) (end 146.855962 93.555038) (width 0.5) (layer "F.Cu") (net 6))
 (segment (start 157.988 89.662) (end 159.795511 91.469511) (width 0.5) (layer "F.Cu") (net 6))
 (segment (start 148.14652 92.26448) (end 154.36952 92.26448) (width 0.5) (layer "F.Cu") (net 6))
 (segment (start 159.512 95.504) (end 158.496 95.504) (width 0.5) (layer "F.Cu") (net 6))
 (segment (start 159.795511 91.469511) (end 159.795511 95.220489) (width 0.5) (layer "F.Cu") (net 6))
 (segment (start 146.855962 93.555038) (end 148.14652 92.26448) (width 0.5) (layer "F.Cu") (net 6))
 (segment (start 159.795511 95.220489) (end 159.512 95.504) (width 0.5) (layer "F.Cu") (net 6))
 (via (at 146.855962 93.589523) (size 0.6) (drill 0.4) (layers "F.Cu" "B.Cu") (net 6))
 (segment (start 146.431 92.15) (end 146.431 93.164561) (width 0.5) (layer "B.Cu") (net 6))
 (segment (start 146.431 93.164561) (end 146.855962 93.589523) (width 0.5) (layer "B.Cu") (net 6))
 (segment (start 151.384 88.12597) (end 152.149816 88.891786) (width 0.5) (layer "F.Cu") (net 7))
 (segment (start 151.384 87.9215) (end 151.384 88.12597) (width 0.5) (layer "F.Cu") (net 7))
 (via (at 152.149816 88.891786) (size 0.6) (drill 0.4) (layers "F.Cu" "B.Cu") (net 7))
 (segment (start 154.051 92.15) (end 154.051 90.79297) (width 0.5) (layer "B.Cu") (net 7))
 (segment (start 154.051 93.599) (end 158.496 98.044) (width 0.5) (layer "B.Cu") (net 7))
 (segment (start 154.051 90.79297) (end 152.149816 88.891786) (width 0.5) (layer "B.Cu") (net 7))
 (segment (start 154.051 92.15) (end 154.051 93.599) (width 0.5) (layer "B.Cu") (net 7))
 (segment (start 143.256 89.408) (end 143.256 91.948) (width 0.5) (layer "F.Cu") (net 8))
 (via (at 143.256 89.408) (size 0.6) (drill 0.4) (layers "F.Cu" "B.Cu") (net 8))
 (via (at 143.256 91.948) (size 0.6) (drill 0.4) (layers "F.Cu" "B.Cu") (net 8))
 (segment (start 155.917479 103.162521) (end 158.496 100.584) (width 0.5) (layer "B.Cu") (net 8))
 (segment (start 142.922479 99.901521) (end 142.922479 101.221991) (width 0.5) (layer "B.Cu") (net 8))
 (segment (start 143.256 99.568) (end 142.922479 99.901521) (width 0.5) (layer "B.Cu") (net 8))
 (segment (start 144.863009 103.162521) (end 155.917479 103.162521) (width 0.5) (layer "B.Cu") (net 8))
 (segment (start 146.431 86.233) (end 143.256 89.408) (width 0.5) (layer "B.Cu") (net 8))
 (segment (start 146.431 85.65) (end 146.431 86.233) (width 0.5) (layer "B.Cu") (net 8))
 (segment (start 143.256 91.948) (end 143.256 99.568) (width 0.5) (layer "B.Cu") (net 8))
 (segment (start 142.922479 101.221991) (end 144.863009 103.162521) (width 0.5) (layer "B.Cu") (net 8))
 (segment (start 149.632858 97.409) (end 147.47373 97.409) (width 0.5) (layer "F.Cu") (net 9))
 (segment (start 151.892 99.668142) (end 149.632858 97.409) (width 0.5) (layer "F.Cu") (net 9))
 (segment (start 147.47373 97.409) (end 144.272 94.20727) (width 0.5) (layer "F.Cu") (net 9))
 (segment (start 151.13 104.394) (end 151.892 103.632) (width 0.5) (layer "F.Cu") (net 9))
 (segment (start 151.892 103.632) (end 151.892 99.668142) (width 0.5) (layer "F.Cu") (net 9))
 (segment (start 144.272 94.20727) (end 144.272 94.107) (width 0.5) (layer "F.Cu") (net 9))
 (via (at 151.13 104.394) (size 0.6) (drill 0.4) (layers "F.Cu" "B.Cu") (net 9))
 (via (at 144.272 94.107) (size 0.6) (drill 0.4) (layers "F.Cu" "B.Cu") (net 9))
 (segment (start 144.272 91.339978) (end 145.927993 89.683985) (width 0.5) (layer "B.Cu") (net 9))
 (segment (start 147.701 85.65) (end 147.586489 85.764511) (width 0.5) (layer "B.Cu") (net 9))
 (segment (start 157.226 104.394) (end 158.496 103.124) (width 0.5) (layer "B.Cu") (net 9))
 (segment (start 147.586489 88.677481) (end 146.579985 89.683985) (width 0.5) (layer "B.Cu") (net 9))
 (segment (start 144.272 91.339978) (end 144.272 93.726) (width 0.5) (layer "B.Cu") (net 9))
 (segment (start 144.272 93.726) (end 144.272 94.107) (width 0.5) (layer "B.Cu") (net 9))
 (segment (start 147.586489 85.764511) (end 147.586489 88.677481) (width 0.5) (layer "B.Cu") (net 9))
 (segment (start 145.927993 89.683985) (end 146.579985 89.683985) (width 0.5) (layer "B.Cu") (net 9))
 (segment (start 151.13 104.394) (end 157.226 104.394) (width 0.5) (layer "B.Cu") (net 9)))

